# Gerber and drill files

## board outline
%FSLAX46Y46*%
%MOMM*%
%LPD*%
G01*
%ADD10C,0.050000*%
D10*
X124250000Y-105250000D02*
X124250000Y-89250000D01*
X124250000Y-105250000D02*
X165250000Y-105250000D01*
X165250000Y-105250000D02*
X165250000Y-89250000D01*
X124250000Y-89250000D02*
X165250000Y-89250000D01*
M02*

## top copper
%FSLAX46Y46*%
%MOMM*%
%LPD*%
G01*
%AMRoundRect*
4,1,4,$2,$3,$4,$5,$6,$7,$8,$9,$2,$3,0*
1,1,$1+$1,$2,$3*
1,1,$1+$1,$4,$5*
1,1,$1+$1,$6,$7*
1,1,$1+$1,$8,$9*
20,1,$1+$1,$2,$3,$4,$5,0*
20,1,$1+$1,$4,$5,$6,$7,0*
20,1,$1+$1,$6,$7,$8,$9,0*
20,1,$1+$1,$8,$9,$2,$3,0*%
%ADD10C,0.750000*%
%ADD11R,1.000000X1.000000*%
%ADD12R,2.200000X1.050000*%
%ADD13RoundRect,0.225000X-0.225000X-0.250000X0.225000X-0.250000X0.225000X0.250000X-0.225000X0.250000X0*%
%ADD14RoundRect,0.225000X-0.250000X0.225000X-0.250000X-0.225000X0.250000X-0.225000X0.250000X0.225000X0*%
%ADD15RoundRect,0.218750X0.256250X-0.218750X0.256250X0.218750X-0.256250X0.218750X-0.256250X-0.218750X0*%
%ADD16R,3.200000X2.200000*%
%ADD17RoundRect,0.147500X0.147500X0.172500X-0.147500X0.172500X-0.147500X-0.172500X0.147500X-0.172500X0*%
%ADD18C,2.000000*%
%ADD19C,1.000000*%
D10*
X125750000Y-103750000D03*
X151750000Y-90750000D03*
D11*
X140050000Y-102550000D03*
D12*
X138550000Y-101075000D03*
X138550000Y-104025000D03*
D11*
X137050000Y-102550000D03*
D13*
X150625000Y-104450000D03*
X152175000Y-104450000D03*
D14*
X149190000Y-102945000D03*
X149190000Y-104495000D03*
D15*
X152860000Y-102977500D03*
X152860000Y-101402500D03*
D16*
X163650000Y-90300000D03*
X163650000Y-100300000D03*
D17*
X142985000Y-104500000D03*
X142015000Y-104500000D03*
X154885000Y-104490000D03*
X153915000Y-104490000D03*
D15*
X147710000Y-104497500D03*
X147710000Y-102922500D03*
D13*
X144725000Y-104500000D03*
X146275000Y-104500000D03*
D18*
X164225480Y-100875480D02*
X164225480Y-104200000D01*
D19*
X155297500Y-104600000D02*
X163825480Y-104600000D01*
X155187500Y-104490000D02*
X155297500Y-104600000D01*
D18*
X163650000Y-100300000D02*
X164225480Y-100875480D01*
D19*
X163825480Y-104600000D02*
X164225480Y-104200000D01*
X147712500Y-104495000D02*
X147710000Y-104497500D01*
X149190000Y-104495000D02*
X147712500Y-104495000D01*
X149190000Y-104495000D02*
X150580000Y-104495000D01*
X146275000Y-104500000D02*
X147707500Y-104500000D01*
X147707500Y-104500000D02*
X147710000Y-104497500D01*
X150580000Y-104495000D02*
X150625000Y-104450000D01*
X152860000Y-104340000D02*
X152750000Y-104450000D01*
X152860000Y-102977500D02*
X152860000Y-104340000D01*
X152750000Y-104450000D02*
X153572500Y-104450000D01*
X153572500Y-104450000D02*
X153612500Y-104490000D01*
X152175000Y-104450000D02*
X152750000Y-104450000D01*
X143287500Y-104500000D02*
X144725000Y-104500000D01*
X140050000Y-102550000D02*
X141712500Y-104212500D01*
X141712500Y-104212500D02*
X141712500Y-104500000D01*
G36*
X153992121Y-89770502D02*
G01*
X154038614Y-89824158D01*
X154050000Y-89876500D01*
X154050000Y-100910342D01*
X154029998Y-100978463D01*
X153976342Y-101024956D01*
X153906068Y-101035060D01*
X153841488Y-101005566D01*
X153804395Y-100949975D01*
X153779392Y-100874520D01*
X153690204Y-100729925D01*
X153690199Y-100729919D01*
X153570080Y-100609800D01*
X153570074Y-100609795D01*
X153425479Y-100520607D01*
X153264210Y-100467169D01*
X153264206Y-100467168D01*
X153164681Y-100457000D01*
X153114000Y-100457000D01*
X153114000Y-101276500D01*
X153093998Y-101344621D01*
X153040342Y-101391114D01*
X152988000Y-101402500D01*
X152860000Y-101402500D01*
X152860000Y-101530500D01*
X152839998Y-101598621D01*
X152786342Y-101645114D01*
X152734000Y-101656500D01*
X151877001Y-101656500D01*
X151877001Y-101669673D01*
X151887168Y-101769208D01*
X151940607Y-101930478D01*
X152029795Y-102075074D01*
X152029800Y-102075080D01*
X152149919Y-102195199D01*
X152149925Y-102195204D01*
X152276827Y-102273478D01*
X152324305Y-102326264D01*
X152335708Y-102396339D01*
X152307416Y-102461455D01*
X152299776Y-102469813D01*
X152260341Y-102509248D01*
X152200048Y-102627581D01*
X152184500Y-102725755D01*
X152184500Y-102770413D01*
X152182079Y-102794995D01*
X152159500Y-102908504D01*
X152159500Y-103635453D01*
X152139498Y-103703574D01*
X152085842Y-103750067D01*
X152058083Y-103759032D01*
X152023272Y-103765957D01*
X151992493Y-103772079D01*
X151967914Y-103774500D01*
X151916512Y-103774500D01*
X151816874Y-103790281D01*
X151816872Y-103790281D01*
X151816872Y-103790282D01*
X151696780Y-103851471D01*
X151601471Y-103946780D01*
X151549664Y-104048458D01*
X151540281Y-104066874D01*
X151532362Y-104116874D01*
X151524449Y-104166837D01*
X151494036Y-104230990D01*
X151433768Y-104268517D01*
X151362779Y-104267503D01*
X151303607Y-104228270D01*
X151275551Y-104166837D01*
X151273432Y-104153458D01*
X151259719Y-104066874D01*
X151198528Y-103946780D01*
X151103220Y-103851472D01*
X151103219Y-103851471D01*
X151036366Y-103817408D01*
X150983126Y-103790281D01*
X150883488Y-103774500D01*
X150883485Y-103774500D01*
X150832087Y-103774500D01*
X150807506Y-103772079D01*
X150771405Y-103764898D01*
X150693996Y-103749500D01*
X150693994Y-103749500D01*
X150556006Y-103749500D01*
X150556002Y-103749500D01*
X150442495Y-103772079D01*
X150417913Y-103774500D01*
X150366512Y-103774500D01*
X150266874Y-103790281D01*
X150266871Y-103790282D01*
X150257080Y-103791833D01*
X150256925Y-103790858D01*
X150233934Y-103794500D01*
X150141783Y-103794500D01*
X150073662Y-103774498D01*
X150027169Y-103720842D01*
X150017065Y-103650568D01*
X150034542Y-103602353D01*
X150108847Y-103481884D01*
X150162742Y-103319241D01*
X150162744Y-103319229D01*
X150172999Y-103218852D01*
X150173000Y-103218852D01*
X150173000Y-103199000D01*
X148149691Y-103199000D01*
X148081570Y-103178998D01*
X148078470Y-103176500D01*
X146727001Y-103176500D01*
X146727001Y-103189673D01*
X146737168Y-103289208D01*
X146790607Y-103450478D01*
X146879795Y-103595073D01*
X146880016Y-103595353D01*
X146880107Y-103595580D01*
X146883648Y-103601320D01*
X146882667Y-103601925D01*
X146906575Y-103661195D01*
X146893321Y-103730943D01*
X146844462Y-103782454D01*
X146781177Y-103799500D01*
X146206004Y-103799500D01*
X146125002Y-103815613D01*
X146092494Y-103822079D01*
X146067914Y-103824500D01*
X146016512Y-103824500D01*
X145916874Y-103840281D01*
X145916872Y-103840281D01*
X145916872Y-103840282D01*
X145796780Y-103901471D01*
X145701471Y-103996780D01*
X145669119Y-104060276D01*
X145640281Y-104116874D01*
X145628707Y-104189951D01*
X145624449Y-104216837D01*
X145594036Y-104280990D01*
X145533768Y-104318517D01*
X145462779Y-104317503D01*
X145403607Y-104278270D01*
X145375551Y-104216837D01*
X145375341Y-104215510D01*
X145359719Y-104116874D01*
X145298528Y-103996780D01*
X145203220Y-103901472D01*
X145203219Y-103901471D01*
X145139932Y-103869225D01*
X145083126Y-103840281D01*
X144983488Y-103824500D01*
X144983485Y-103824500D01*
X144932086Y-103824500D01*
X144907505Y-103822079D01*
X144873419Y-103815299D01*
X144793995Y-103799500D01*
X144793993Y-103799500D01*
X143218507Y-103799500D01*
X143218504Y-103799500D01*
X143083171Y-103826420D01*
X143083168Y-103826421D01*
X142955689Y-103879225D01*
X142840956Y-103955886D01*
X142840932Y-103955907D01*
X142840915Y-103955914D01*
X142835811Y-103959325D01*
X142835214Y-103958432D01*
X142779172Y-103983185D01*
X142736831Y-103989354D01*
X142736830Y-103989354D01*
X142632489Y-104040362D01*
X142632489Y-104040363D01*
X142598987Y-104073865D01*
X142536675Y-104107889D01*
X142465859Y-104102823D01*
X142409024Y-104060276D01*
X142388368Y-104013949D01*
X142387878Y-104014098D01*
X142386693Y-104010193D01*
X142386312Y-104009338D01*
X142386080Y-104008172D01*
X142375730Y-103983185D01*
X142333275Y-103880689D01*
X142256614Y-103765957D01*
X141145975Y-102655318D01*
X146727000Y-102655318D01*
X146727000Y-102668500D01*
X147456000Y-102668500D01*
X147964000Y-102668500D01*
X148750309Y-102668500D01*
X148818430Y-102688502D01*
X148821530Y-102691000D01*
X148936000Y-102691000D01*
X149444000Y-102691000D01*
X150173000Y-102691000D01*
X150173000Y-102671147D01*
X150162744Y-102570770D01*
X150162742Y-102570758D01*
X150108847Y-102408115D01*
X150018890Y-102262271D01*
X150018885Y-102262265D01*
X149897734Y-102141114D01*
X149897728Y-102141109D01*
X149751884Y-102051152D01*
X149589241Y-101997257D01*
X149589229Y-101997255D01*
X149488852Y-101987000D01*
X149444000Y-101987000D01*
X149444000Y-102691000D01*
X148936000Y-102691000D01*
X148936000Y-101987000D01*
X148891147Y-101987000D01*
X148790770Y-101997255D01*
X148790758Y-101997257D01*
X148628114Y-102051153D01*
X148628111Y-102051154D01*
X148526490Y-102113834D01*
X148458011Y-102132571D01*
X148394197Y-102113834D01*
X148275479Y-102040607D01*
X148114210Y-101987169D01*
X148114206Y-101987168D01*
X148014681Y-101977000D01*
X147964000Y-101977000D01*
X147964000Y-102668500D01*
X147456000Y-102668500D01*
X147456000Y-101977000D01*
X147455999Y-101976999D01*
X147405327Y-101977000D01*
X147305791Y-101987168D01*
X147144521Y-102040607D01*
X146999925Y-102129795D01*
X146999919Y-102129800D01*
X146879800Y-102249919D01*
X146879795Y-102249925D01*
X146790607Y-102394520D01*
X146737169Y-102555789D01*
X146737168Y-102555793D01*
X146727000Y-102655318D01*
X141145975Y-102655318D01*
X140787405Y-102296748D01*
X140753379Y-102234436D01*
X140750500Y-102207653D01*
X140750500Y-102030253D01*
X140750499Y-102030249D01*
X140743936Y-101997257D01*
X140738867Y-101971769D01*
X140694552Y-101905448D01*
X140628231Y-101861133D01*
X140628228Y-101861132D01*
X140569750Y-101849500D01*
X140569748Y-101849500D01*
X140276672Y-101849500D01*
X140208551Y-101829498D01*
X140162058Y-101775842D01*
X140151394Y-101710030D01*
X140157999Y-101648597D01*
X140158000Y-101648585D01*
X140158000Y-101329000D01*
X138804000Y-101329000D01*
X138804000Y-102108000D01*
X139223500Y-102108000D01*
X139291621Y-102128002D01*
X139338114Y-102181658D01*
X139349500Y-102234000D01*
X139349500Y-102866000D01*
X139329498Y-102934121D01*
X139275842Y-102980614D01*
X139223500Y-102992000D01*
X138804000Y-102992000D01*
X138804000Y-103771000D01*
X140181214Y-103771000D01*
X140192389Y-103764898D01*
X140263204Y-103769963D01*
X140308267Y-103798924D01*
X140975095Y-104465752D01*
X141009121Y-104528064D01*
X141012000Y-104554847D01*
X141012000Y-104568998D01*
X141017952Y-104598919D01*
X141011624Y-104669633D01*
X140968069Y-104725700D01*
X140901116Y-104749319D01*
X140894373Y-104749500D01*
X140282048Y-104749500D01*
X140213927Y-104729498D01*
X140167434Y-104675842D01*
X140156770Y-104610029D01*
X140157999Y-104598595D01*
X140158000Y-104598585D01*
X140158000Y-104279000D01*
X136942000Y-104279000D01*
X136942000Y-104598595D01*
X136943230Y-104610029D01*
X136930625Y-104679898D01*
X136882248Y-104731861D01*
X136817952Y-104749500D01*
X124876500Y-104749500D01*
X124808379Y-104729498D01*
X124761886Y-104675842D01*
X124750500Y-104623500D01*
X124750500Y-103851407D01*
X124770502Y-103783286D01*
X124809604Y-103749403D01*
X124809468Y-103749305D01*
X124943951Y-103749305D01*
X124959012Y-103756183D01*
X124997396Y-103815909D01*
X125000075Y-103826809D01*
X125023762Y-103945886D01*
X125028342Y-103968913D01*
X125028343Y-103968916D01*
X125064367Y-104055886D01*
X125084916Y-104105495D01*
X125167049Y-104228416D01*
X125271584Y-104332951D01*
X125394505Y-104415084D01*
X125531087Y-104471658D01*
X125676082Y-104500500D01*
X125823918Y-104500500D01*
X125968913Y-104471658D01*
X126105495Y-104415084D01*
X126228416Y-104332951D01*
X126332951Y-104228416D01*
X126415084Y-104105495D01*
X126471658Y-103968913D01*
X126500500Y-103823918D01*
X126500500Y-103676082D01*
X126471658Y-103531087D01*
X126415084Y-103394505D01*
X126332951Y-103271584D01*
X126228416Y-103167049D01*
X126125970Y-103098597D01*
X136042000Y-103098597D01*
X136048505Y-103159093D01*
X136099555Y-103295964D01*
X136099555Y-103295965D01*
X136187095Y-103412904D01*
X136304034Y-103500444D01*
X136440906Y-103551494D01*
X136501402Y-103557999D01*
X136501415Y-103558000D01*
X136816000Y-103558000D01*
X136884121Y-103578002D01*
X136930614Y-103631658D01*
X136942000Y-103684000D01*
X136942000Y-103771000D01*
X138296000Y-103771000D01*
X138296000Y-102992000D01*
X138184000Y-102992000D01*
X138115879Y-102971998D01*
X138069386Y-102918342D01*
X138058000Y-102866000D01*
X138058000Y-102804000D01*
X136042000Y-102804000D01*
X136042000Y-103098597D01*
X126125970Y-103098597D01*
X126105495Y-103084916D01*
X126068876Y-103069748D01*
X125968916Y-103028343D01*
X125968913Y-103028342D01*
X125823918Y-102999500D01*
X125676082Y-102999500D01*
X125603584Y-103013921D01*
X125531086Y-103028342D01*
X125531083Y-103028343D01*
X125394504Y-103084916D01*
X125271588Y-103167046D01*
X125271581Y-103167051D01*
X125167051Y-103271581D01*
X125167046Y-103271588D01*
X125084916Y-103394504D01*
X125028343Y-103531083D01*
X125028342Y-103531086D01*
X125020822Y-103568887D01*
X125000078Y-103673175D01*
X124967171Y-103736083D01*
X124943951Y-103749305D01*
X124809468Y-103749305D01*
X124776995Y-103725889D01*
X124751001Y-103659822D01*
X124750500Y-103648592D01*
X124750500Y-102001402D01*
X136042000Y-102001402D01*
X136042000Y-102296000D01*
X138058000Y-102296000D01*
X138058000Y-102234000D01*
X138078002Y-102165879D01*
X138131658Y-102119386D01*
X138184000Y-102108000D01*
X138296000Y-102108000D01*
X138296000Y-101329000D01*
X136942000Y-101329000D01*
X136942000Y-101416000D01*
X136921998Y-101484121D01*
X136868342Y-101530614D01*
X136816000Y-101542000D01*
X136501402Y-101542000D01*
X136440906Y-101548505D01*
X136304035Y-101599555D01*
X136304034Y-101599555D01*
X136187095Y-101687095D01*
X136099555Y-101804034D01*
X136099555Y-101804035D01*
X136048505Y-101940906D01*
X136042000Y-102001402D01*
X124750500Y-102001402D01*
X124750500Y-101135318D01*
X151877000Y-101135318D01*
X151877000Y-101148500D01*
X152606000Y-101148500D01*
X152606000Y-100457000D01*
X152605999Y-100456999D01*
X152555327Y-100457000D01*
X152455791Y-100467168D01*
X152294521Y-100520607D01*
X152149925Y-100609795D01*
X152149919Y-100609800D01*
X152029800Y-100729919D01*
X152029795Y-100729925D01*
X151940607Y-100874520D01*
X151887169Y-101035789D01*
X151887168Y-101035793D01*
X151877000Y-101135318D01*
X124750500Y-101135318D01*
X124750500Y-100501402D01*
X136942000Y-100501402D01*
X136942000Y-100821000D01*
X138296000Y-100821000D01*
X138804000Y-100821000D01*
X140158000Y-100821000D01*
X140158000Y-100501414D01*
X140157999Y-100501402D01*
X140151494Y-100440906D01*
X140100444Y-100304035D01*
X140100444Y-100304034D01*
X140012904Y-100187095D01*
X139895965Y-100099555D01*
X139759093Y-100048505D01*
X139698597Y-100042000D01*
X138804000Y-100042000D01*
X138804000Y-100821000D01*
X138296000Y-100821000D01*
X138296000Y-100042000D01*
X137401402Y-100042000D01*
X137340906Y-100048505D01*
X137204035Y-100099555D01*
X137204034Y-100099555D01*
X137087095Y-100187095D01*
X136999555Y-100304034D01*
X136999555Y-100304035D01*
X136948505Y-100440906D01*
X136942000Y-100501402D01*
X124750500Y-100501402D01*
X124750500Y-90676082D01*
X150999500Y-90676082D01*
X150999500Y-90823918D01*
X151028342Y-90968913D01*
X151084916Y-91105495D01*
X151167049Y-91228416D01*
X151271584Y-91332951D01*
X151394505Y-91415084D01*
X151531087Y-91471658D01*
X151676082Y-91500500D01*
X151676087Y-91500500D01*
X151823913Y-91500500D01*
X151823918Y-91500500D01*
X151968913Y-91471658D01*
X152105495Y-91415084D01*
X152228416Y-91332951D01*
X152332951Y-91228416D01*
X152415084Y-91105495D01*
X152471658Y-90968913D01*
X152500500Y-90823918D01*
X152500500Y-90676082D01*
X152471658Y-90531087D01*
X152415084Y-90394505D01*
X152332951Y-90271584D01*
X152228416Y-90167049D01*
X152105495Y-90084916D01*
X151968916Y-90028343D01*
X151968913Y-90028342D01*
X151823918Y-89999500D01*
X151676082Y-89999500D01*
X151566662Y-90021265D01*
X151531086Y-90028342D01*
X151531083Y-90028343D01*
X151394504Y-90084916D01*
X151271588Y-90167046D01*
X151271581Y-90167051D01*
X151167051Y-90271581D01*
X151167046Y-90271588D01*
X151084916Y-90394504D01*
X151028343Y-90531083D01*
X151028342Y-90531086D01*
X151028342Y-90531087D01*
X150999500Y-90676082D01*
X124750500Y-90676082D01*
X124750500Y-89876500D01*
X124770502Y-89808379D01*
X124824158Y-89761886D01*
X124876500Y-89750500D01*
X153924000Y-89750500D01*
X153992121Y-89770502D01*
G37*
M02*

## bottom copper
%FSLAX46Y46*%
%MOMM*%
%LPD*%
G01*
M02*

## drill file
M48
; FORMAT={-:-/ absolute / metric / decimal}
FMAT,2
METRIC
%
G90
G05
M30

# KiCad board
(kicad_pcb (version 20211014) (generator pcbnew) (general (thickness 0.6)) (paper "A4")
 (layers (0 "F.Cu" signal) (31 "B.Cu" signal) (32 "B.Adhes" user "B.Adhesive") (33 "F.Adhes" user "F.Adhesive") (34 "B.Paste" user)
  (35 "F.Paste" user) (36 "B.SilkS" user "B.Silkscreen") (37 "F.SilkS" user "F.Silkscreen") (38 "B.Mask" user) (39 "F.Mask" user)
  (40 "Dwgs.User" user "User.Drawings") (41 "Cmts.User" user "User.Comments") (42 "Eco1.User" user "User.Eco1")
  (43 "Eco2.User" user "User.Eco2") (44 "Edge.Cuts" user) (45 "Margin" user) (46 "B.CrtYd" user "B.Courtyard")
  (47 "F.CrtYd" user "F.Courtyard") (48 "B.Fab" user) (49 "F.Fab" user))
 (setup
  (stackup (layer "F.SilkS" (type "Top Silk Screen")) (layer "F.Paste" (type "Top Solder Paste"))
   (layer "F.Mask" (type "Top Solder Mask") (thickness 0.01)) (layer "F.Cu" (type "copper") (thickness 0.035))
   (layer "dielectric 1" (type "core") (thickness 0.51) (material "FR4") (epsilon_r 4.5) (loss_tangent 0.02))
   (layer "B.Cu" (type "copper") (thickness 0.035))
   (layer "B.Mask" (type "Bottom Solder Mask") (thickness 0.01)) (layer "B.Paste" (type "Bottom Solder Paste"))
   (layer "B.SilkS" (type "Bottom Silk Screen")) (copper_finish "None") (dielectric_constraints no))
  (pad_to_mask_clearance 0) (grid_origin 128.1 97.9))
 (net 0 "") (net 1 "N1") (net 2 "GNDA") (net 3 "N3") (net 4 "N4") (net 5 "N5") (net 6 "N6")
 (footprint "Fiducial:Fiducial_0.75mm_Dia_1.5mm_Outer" (layer "F.Cu") (at 125.75 103.75)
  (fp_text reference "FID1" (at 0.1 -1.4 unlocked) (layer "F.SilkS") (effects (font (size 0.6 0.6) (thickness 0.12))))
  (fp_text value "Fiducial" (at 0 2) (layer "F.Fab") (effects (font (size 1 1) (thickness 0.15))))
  (pad "" smd circle locked (at 0 0) (size 0.75 0.75) (layers "F.Cu" "F.Mask") (solder_mask_margin 0.375) (clearance 0.375)))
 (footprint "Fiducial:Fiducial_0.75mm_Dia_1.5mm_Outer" (layer "F.Cu") (at 151.75 90.75)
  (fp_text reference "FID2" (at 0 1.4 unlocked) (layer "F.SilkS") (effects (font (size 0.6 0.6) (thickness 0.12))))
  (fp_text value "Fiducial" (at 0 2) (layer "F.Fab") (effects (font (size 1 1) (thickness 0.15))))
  (pad "" smd circle locked (at 0 0) (size 0.75 0.75) (layers "F.Cu" "F.Mask") (solder_mask_margin 0.375) (clearance 0.375)))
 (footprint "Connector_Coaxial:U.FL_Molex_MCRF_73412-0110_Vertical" (layer "F.Cu") (at 138.55 102.55 90)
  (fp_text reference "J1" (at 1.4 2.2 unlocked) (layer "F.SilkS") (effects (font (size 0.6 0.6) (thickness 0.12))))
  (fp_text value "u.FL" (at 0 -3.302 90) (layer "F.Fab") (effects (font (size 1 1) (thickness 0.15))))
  (pad "1" smd rect locked (at 0 1.5 90) (size 1 1) (layers "F.Cu" "F.Paste" "F.Mask") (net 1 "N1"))
  (pad "2" smd rect locked (at 1.475 0 90) (size 1.05 2.2) (layers "F.Cu" "F.Paste" "F.Mask") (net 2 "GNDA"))
  (pad "2" smd rect locked (at -1.475 0 90) (size 1.05 2.2) (layers "F.Cu" "F.Paste" "F.Mask") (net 2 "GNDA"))
  (pad "2" smd rect locked (at 0 -1.5 90) (size 1 1) (layers "F.Cu" "F.Paste" "F.Mask") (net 2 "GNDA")))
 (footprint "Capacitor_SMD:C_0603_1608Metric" (layer "F.Cu") (at 151.4 104.45)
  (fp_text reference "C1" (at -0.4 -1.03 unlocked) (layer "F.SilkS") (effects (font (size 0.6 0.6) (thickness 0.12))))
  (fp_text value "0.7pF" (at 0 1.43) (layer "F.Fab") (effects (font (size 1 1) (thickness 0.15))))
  (pad "1" smd roundrect locked (at -0.775 0) (size 0.9 0.95) (layers "F.Cu" "F.Paste" "F.Mask") (roundrect_rratio 0.25) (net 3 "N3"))
  (pad "2" smd roundrect locked (at 0.775 0) (size 0.9 0.95) (layers "F.Cu" "F.Paste" "F.Mask") (roundrect_rratio 0.25) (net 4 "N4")))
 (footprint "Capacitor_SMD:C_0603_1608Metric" (layer "F.Cu") (at 149.19 103.72 -90)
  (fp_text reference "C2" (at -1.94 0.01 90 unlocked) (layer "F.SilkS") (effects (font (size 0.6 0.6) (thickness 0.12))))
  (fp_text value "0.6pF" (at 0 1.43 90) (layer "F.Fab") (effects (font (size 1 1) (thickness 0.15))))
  (pad "1" smd roundrect locked (at -0.775 0 270) (size 0.9 0.95) (layers "F.Cu" "F.Paste" "F.Mask") (roundrect_rratio 0.25) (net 2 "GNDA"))
  (pad "2" smd roundrect locked (at 0.775 0 270) (size 0.9 0.95) (layers "F.Cu" "F.Paste" "F.Mask") (roundrect_rratio 0.25) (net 3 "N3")))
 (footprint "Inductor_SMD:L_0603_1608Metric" (layer "F.Cu") (at 152.86 102.19 90)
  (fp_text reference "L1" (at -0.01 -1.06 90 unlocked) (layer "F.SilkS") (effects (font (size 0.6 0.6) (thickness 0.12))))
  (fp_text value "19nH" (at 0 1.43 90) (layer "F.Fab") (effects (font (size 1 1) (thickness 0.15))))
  (pad "1" smd roundrect locked (at -0.7875 0 90) (size 0.875 0.95) (layers "F.Cu" "F.Paste" "F.Mask") (roundrect_rratio 0.25) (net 4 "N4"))
  (pad "2" smd roundrect locked (at 0.7875 0 90) (size 0.875 0.95) (layers "F.Cu" "F.Paste" "F.Mask") (roundrect_rratio 0.25) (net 2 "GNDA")))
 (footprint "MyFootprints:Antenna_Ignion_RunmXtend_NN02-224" (layer "F.Cu") (at 163.65 95.3 -90)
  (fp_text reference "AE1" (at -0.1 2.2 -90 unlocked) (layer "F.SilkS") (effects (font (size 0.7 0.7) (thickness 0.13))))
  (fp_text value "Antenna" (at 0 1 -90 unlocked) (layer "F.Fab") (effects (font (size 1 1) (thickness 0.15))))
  (pad "" smd rect (at -5 0 270) (size 2.2 3.2) (layers "F.Cu" "F.Paste" "F.Mask"))
  (pad "1" smd rect (at 5 0 270) (size 2.2 3.2) (layers "F.Cu" "F.Paste" "F.Mask") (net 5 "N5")))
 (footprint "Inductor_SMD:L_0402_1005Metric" (layer "F.Cu") (at 142.5 104.5 180)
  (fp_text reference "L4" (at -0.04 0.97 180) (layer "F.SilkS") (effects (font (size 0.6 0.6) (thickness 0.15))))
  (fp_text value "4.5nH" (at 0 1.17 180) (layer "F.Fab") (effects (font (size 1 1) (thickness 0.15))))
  (pad "1" smd roundrect locked (at -0.485 0 180) (size 0.59 0.64) (layers "F.Cu" "F.Paste" "F.Mask") (roundrect_rratio 0.25) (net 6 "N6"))
  (pad "2" smd roundrect locked (at 0.485 0 180) (size 0.59 0.64) (layers "F.Cu" "F.Paste" "F.Mask") (roundrect_rratio 0.25) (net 1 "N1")))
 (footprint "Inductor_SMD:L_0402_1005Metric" (layer "F.Cu") (at 154.4 104.49 180)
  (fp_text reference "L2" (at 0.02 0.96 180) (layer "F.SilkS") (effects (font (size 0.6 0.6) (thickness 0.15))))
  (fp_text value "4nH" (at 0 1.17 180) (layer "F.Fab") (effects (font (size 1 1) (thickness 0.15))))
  (pad "1" smd roundrect locked (at -0.485 0 180) (size 0.59 0.64) (layers "F.Cu" "F.Paste" "F.Mask") (roundrect_rratio 0.25) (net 5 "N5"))
  (pad "2" smd roundrect locked (at 0.485 0 180) (size 0.59 0.64) (layers "F.Cu" "F.Paste" "F.Mask") (roundrect_rratio 0.25) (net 4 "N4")))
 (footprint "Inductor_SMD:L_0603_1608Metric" (layer "F.Cu") (at 147.71 103.71 90)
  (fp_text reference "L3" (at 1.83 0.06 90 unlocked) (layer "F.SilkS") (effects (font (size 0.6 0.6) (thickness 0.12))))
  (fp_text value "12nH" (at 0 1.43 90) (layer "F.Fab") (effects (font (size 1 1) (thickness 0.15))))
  (pad "1" smd roundrect locked (at -0.7875 0 90) (size 0.875 0.95) (layers "F.Cu" "F.Paste" "F.Mask") (roundrect_rratio 0.25) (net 3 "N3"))
  (pad "2" smd roundrect locked (at 0.7875 0 90) (size 0.875 0.95) (layers "F.Cu" "F.Paste" "F.Mask") (roundrect_rratio 0.25) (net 2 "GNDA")))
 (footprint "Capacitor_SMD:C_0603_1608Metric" (layer "F.Cu") (at 145.5 104.5)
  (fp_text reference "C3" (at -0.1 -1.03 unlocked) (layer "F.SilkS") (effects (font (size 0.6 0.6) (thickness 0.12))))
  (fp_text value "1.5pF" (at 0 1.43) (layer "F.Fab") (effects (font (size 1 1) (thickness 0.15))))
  (pad "1" smd roundrect locked (at -0.775 0) (size 0.9 0.95) (layers "F.Cu" "F.Paste" "F.Mask") (roundrect_rratio 0.25) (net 6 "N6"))
  (pad "2" smd roundrect locked (at 0.775 0) (size 0.9 0.95) (layers "F.Cu" "F.Paste" "F.Mask") (roundrect_rratio 0.25) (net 3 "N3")))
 (gr_line (start 124.25 105.25) (end 124.25 89.25) (layer "Edge.Cuts") (width 0.05))
 (gr_line (start 124.25 105.25) (end 165.25 105.25) (layer "Edge.Cuts") (width 0.05))
 (gr_line (start 165.25 105.25) (end 165.25 89.25) (layer "Edge.Cuts") (width 0.05))
 (gr_line (start 124.25 89.25) (end 165.25 89.25) (layer "Edge.Cuts") (width 0.05))
 (segment (start 164.22548 100.87548) (end 164.22548 104.2) (width 2) (layer "F.Cu") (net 5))
 (segment (start 155.2975 104.6) (end 163.82548 104.6) (width 1) (layer "F.Cu") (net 5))
 (segment (start 155.1875 104.49) (end 155.2975 104.6) (width 1) (layer "F.Cu") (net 5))
 (segment (start 163.65 100.3) (end 164.22548 100.87548) (width 2) (layer "F.Cu") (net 5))
 (segment (start 163.82548 104.6) (end 164.22548 104.2) (width 1) (layer "F.Cu") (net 5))
 (segment (start 147.7125 104.495) (end 147.71 104.4975) (width 1) (layer "F.Cu") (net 3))
 (segment (start 149.19 104.495) (end 147.7125 104.495) (width 1) (layer "F.Cu") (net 3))
 (segment (start 149.19 104.495) (end 150.58 104.495) (width 1) (layer "F.Cu") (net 3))
 (segment (start 146.275 104.5) (end 147.7075 104.5) (width 1) (layer "F.Cu") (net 3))
 (segment (start 147.7075 104.5) (end 147.71 104.4975) (width 1) (layer "F.Cu") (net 3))
 (segment (start 150.58 104.495) (end 150.625 104.45) (width 1) (layer "F.Cu") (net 3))
 (segment (start 152.86 104.34) (end 152.75 104.45) (width 1) (layer "F.Cu") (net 4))
 (segment (start 152.86 102.9775) (end 152.86 104.34) (width 1) (layer "F.Cu") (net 4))
 (segment (start 152.75 104.45) (end 153.5725 104.45) (width 1) (layer "F.Cu") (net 4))
 (segment (start 153.5725 104.45) (end 153.6125 104.49) (width 1) (layer "F.Cu") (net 4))
 (segment (start 152.175 104.45) (end 152.75 104.45) (width 1) (layer "F.Cu") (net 4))
 (segment (start 143.2875 104.5) (end 144.725 104.5) (width 1) (layer "F.Cu") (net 6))
 (segment (start 140.05 102.55) (end 141.7125 104.2125) (width 1) (layer "F.Cu") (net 1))
 (segment (start 141.7125 104.2125) (end 141.7125 104.5) (width 1) (layer "F.Cu") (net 1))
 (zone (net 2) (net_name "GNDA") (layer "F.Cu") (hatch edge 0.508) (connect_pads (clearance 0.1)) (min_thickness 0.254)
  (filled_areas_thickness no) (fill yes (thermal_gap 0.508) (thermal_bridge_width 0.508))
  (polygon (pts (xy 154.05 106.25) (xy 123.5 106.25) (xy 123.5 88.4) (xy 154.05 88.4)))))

